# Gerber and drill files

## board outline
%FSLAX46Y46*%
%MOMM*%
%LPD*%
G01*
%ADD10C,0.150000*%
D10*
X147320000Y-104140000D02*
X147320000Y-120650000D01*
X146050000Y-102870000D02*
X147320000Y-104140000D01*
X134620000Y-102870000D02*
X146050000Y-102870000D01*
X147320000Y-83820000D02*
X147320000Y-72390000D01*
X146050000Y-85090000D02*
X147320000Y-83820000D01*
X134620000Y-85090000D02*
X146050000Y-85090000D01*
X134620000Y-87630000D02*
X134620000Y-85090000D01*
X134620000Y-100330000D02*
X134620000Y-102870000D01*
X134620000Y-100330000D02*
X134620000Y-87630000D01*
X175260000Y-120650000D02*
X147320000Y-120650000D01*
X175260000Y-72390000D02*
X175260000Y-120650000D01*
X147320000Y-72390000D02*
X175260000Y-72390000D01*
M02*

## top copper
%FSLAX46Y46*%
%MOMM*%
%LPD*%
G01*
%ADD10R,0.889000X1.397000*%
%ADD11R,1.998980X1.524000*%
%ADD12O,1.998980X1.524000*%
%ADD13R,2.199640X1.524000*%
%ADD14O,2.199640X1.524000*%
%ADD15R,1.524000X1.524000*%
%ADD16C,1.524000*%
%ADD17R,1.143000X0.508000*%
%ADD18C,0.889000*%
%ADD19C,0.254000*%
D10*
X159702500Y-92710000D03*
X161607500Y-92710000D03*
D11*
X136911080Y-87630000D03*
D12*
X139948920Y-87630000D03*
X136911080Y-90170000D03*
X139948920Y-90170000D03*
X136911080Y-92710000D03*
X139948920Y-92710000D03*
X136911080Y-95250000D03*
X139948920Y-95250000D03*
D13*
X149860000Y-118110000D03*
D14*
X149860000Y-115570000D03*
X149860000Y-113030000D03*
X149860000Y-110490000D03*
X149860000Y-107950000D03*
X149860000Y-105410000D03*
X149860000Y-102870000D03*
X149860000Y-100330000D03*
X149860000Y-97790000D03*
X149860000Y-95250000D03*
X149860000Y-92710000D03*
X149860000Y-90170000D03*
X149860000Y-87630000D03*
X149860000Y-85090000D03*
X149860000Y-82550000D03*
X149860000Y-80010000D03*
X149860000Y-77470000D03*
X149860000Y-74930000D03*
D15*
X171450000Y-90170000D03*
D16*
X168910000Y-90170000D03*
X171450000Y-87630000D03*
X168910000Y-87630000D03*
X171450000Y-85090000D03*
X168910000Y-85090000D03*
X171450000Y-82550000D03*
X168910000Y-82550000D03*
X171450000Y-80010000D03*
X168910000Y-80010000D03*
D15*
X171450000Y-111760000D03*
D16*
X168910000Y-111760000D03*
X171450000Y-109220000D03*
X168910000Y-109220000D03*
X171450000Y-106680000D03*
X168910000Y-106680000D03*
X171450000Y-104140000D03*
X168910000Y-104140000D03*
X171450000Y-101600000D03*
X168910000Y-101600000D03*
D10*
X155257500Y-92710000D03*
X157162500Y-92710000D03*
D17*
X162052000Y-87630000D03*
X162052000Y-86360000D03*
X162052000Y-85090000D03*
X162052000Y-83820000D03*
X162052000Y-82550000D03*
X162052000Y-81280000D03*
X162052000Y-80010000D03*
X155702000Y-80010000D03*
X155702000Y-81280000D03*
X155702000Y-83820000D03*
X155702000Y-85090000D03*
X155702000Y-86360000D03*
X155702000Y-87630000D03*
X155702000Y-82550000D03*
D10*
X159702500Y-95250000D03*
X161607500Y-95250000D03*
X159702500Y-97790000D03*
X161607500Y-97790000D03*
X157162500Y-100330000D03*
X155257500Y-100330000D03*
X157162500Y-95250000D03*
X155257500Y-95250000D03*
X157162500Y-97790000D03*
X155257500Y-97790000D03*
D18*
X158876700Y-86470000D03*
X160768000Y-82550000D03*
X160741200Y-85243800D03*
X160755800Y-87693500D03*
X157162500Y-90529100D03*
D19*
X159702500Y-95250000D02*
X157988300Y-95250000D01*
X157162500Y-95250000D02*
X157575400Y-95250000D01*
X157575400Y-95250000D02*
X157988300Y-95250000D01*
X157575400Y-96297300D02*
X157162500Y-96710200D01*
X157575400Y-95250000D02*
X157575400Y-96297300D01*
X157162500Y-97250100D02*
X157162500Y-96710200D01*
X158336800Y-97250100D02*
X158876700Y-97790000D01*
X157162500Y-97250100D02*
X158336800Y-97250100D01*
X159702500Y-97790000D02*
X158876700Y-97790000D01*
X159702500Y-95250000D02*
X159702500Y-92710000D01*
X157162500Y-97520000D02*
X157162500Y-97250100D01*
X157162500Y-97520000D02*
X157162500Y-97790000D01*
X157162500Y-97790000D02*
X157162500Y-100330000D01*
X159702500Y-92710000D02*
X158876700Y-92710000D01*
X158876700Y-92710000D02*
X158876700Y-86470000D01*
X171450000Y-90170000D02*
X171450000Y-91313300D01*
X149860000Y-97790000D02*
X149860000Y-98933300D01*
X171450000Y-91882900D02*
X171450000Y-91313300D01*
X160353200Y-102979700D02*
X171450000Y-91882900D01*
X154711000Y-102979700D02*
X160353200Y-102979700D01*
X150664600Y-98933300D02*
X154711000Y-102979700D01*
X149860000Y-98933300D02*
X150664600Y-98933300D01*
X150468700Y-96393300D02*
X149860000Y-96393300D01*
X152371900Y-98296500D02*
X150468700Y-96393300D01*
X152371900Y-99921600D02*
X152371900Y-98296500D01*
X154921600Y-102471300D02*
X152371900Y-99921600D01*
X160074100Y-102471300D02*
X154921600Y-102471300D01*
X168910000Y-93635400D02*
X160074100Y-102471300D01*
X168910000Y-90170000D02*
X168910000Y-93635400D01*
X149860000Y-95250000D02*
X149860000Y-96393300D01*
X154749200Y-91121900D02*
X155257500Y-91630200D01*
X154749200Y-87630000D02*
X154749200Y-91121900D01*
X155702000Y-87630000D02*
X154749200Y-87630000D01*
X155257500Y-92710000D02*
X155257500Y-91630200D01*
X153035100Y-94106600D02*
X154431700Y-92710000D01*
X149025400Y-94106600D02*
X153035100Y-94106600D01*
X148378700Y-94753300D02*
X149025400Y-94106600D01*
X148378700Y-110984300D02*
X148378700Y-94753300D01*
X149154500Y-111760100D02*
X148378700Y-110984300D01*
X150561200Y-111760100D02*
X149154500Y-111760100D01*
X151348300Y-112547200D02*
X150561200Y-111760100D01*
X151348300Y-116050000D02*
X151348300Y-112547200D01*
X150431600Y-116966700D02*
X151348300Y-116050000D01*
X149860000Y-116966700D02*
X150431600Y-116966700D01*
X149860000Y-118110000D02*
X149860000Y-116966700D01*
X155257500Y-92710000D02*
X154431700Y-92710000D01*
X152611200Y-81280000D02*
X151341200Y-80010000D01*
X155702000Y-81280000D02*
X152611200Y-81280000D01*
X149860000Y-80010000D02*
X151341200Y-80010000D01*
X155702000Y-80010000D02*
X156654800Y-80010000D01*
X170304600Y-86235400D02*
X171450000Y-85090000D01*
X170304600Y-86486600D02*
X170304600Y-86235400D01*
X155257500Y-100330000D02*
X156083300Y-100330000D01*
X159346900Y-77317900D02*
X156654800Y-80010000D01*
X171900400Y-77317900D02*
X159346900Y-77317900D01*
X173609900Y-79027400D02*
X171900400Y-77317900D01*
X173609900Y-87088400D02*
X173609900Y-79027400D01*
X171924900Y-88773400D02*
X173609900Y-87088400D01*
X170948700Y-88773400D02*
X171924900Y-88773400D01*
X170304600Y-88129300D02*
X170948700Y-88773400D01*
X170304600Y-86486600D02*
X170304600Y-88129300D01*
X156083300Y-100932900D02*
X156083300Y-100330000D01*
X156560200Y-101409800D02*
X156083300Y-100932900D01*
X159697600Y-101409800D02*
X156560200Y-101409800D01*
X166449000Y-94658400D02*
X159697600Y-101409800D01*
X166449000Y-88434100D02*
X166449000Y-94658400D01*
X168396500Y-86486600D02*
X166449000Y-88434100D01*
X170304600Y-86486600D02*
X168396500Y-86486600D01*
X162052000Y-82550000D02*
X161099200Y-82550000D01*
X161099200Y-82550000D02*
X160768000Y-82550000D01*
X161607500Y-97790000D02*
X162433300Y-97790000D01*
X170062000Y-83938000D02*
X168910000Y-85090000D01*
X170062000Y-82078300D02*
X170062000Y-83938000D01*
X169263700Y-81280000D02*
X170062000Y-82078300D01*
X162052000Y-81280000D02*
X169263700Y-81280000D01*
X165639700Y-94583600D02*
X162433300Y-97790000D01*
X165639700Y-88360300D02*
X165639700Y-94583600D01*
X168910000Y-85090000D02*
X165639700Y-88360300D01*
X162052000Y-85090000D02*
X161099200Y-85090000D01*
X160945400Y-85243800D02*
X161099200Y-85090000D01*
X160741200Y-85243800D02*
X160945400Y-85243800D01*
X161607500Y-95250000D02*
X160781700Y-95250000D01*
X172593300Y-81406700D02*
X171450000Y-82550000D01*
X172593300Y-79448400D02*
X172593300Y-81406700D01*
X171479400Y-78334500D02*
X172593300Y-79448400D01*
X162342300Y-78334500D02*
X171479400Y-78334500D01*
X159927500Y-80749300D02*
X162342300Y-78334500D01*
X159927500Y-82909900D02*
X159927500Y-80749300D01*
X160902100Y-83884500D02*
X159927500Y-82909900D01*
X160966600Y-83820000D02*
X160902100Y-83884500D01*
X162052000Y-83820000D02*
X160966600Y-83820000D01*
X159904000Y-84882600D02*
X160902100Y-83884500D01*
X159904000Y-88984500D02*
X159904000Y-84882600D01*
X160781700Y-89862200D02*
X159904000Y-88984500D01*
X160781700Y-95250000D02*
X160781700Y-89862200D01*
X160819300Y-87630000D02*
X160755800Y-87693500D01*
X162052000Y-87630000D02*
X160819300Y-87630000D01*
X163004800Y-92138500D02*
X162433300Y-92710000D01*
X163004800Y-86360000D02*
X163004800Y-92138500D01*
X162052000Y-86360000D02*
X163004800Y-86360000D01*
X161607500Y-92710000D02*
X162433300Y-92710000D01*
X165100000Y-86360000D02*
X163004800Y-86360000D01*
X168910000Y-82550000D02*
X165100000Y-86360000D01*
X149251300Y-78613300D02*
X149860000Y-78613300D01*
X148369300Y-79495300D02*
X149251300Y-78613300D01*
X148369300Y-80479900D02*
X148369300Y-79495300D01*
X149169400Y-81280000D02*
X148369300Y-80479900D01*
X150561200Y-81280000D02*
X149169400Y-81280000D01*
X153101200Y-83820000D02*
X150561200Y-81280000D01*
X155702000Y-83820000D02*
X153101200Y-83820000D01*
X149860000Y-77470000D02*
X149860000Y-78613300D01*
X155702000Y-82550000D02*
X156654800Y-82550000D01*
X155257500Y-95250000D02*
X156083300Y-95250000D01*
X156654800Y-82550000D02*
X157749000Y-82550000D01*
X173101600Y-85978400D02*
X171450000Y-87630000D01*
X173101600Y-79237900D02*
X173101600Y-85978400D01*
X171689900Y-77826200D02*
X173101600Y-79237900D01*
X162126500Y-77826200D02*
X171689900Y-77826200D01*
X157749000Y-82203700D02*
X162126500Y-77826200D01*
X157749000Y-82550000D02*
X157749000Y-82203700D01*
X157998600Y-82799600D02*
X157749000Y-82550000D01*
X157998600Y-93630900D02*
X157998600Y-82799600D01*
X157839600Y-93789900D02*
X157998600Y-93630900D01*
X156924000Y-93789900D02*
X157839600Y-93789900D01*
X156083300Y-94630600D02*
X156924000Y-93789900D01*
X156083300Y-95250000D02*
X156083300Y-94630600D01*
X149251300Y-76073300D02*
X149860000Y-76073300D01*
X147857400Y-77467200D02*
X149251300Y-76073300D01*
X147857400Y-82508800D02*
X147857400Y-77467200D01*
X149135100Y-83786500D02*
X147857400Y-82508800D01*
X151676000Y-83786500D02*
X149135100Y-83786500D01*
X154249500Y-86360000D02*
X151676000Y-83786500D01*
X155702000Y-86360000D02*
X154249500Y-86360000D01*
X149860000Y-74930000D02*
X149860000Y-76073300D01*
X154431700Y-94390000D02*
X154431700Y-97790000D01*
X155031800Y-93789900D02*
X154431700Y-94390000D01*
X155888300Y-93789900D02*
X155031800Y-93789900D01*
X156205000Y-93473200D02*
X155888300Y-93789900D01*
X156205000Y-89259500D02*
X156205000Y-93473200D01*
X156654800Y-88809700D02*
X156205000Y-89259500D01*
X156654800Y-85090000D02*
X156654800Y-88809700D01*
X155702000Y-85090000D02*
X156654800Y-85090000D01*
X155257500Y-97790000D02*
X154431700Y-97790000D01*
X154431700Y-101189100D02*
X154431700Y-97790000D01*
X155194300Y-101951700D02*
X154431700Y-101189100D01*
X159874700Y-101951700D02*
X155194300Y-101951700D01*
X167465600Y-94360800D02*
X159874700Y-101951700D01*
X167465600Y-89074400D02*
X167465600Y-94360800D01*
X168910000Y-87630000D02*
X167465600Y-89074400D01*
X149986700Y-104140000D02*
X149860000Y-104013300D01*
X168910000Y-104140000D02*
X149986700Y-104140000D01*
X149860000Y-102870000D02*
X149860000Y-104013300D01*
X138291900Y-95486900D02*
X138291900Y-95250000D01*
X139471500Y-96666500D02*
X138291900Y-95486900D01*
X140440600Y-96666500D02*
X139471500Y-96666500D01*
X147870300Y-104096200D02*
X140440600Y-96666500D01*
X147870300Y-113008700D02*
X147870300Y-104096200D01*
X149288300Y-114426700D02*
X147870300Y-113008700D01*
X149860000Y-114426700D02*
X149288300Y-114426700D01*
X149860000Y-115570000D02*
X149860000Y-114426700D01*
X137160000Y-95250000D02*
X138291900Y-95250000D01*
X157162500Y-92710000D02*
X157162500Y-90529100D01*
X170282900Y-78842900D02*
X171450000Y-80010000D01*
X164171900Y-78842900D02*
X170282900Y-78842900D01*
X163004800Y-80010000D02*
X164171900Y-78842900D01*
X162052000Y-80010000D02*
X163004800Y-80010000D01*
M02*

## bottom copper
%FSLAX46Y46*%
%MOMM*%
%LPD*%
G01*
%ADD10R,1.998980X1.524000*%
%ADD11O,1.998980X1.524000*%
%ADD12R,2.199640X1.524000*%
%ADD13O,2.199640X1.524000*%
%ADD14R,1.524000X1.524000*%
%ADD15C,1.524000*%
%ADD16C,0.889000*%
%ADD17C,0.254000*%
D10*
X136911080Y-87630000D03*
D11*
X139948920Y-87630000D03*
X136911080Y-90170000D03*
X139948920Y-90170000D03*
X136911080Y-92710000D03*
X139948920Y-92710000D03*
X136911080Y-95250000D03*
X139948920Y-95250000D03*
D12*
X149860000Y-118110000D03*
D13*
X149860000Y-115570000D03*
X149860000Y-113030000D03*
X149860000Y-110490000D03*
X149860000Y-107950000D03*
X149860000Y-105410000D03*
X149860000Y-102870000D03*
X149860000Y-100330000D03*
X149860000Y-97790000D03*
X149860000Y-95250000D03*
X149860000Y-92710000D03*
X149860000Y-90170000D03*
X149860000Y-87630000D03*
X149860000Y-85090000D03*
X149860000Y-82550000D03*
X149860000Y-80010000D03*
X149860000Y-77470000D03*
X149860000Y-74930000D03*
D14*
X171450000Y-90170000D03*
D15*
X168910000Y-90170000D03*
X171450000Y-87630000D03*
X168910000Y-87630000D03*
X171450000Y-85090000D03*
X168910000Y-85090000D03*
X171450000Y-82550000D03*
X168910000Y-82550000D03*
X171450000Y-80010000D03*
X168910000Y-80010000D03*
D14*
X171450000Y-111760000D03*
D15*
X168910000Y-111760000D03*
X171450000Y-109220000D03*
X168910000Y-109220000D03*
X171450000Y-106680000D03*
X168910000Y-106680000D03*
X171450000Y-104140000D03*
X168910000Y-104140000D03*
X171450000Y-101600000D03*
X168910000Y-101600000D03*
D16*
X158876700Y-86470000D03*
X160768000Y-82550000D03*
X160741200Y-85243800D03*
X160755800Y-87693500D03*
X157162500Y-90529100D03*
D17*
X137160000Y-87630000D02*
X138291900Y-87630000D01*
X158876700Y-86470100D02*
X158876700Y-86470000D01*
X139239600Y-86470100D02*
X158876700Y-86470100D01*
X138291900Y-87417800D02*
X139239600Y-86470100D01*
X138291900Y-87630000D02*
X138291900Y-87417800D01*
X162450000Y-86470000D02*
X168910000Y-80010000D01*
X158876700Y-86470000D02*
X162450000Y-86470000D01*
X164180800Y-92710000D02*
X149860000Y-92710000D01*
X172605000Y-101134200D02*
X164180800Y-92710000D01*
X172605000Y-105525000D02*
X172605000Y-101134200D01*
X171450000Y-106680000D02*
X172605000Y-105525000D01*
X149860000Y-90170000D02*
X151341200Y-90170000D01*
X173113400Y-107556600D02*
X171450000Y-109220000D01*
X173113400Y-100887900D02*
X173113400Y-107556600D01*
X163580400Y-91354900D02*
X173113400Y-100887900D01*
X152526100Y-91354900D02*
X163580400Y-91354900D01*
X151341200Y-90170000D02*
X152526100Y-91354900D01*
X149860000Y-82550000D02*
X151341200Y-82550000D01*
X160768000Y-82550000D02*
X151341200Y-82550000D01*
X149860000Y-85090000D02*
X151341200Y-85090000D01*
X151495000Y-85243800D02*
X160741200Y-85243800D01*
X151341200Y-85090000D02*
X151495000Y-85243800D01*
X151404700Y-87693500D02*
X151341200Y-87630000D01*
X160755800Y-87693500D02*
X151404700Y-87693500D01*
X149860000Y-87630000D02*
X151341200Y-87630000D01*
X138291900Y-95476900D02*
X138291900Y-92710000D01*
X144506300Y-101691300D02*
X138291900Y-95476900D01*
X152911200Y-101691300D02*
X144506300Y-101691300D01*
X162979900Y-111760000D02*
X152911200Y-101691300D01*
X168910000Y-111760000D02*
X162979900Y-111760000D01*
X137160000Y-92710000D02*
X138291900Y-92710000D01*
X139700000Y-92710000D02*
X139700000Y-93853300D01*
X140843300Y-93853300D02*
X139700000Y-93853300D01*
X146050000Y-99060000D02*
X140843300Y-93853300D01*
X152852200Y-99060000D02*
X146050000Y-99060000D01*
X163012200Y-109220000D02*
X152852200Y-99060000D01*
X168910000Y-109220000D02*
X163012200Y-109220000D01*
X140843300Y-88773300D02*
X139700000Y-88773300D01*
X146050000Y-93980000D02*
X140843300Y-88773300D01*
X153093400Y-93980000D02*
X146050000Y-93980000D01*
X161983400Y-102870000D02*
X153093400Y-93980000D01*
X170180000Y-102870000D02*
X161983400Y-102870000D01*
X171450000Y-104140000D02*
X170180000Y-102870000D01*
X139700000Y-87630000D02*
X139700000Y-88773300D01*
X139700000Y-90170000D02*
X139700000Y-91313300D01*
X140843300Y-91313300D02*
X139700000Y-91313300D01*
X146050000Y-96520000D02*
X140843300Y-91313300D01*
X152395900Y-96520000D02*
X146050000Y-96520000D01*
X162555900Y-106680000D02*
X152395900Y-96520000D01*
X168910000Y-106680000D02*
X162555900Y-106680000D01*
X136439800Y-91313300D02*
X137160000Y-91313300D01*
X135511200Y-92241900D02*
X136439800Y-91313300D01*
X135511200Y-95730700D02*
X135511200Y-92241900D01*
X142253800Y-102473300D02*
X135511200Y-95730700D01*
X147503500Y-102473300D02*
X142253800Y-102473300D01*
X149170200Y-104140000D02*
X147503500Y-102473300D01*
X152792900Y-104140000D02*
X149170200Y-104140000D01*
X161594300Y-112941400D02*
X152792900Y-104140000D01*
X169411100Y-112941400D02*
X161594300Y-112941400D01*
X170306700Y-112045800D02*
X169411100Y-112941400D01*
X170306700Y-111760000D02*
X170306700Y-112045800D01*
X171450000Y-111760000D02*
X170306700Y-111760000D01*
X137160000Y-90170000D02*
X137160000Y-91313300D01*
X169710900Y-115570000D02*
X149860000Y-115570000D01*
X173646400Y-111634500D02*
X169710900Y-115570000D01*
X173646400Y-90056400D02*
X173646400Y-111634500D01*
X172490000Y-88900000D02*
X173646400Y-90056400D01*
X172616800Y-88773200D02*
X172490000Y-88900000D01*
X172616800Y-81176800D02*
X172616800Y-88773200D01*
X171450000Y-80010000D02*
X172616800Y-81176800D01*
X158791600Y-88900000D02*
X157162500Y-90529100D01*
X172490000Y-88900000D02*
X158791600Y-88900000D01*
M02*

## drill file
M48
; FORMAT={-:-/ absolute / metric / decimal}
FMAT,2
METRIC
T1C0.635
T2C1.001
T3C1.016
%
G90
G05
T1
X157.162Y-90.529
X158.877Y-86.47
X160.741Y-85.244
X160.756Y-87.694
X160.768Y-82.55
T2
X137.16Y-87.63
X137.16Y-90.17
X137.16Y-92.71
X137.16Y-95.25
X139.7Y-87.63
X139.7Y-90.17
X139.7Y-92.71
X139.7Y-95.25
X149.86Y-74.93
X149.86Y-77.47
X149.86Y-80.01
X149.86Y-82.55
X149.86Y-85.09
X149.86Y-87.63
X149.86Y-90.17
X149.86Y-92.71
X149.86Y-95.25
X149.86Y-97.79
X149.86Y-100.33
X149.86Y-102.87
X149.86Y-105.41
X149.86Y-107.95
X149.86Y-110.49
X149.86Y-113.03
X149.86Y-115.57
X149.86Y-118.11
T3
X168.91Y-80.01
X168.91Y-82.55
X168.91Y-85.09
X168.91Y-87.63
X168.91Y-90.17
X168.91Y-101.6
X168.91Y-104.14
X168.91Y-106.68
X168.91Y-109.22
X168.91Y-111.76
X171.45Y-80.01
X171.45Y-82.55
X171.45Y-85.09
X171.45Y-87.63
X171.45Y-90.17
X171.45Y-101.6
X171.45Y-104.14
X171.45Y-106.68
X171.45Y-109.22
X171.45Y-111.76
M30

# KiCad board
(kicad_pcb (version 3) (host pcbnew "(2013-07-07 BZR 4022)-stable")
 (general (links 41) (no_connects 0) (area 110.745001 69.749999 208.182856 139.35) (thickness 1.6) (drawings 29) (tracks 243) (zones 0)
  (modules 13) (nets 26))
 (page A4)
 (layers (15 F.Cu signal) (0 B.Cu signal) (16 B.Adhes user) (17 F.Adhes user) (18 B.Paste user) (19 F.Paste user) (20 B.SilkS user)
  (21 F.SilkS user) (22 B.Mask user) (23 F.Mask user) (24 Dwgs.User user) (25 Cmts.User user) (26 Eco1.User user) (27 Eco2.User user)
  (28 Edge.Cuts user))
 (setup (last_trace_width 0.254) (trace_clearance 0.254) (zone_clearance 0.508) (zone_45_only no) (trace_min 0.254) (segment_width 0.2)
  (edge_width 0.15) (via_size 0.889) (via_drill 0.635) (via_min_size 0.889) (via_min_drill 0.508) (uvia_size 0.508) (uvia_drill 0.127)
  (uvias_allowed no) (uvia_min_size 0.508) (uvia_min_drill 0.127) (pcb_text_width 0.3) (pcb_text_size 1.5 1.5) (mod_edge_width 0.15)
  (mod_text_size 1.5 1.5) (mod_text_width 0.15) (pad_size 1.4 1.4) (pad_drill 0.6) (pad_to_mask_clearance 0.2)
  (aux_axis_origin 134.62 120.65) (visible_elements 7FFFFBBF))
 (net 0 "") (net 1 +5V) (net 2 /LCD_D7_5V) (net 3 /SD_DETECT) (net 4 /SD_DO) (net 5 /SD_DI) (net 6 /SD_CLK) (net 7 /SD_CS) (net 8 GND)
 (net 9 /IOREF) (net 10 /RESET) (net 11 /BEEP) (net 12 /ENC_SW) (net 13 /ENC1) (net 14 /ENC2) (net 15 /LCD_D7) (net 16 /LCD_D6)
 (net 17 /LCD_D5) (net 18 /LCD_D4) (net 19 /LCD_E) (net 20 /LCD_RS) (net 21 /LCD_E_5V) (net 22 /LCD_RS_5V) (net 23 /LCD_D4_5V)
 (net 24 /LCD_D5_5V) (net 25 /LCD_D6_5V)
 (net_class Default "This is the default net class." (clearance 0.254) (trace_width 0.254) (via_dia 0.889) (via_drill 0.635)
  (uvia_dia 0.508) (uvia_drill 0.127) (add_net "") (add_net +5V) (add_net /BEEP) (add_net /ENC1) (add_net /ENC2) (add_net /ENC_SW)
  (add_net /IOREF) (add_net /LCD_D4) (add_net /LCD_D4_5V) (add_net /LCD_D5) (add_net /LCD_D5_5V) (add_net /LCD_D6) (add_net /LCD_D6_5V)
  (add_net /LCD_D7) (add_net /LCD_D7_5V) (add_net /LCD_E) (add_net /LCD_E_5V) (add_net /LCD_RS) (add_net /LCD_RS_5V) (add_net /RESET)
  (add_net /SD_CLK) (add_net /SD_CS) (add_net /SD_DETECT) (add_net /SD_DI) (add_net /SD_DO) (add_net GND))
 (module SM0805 (layer F.Cu) (at 160.655 92.71)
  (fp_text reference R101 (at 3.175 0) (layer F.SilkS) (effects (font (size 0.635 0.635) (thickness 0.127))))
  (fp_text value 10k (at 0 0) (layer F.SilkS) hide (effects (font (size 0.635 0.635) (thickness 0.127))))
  (pad 1 smd rect (at -0.9525 0) (size 0.889 1.397) (layers F.Cu F.Paste F.Mask) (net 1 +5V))
  (pad 2 smd rect (at 0.9525 0) (size 0.889 1.397) (layers F.Cu F.Paste F.Mask) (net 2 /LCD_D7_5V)))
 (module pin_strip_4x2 (layer F.Cu) (at 138.43 91.44 270)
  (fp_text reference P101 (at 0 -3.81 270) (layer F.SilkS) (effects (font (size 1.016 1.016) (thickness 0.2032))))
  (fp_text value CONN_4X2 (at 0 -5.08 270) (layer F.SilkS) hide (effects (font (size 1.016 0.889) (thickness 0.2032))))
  (pad 1 thru_hole rect (at -3.81 1.27 270) (size 1.524 1.99898) (drill 1.00076 (offset 0 0.24892)) (layers *.Cu *.Mask F.SilkS) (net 1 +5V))
  (pad 2 thru_hole oval (at -3.81 -1.27 270) (size 1.524 1.99898) (drill 1.00076 (offset 0 -0.24892)) (layers *.Cu *.Mask F.SilkS)
   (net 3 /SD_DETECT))
  (pad 3 thru_hole oval (at -1.27 1.27 270) (size 1.524 1.99898) (drill 1.00076 (offset 0 0.24892)) (layers *.Cu *.Mask F.SilkS)
   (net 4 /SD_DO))
  (pad 4 thru_hole oval (at -1.27 -1.27 270) (size 1.524 1.99898) (drill 1.00076 (offset 0 -0.24892)) (layers *.Cu *.Mask F.SilkS)
   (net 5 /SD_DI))
  (pad 5 thru_hole oval (at 1.27 1.27 270) (size 1.524 1.99898) (drill 1.00076 (offset 0 0.24892)) (layers *.Cu *.Mask F.SilkS)
   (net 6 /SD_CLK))
  (pad 6 thru_hole oval (at 1.27 -1.27 270) (size 1.524 1.99898) (drill 1.00076 (offset 0 -0.24892)) (layers *.Cu *.Mask F.SilkS)
   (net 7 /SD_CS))
  (pad 7 thru_hole oval (at 3.81 1.27 270) (size 1.524 1.99898) (drill 1.00076 (offset 0 0.24892)) (layers *.Cu *.Mask F.SilkS) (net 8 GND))
  (pad 8 thru_hole oval (at 3.81 -1.27 270) (size 1.524 1.99898) (drill 1.00076 (offset 0 -0.24892)) (layers *.Cu *.Mask F.SilkS)))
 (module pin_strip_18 (layer B.Cu) (at 149.86 96.52 90)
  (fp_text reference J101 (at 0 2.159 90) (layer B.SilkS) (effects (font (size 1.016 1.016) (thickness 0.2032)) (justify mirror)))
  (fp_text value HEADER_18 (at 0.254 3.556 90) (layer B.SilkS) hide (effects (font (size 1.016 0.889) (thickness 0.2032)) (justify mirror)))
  (pad 1 thru_hole rect (at -21.59 0 90) (size 1.524 2.19964) (drill 1.00076) (layers *.Cu *.Mask B.SilkS) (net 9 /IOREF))
  (pad 2 thru_hole oval (at -19.05 0 90) (size 1.524 2.19964) (drill 1.00076) (layers *.Cu *.Mask B.SilkS) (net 8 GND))
  (pad 3 thru_hole oval (at -16.51 0 90) (size 1.524 2.19964) (drill 1.00076) (layers *.Cu *.Mask B.SilkS))
  (pad 4 thru_hole oval (at -13.97 0 90) (size 1.524 2.19964) (drill 1.00076) (layers *.Cu *.Mask B.SilkS))
  (pad 5 thru_hole oval (at -11.43 0 90) (size 1.524 2.19964) (drill 1.00076) (layers *.Cu *.Mask B.SilkS))
  (pad 6 thru_hole oval (at -8.89 0 90) (size 1.524 2.19964) (drill 1.00076) (layers *.Cu *.Mask B.SilkS))
  (pad 7 thru_hole oval (at -6.35 0 90) (size 1.524 2.19964) (drill 1.00076) (layers *.Cu *.Mask B.SilkS) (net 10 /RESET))
  (pad 8 thru_hole oval (at -3.81 0 90) (size 1.524 2.19964) (drill 1.00076) (layers *.Cu *.Mask B.SilkS))
  (pad 9 thru_hole oval (at -1.27 0 90) (size 1.524 2.19964) (drill 1.00076) (layers *.Cu *.Mask B.SilkS) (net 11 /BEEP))
  (pad 10 thru_hole oval (at 1.27 0 90) (size 1.524 2.19964) (drill 1.00076) (layers *.Cu *.Mask B.SilkS) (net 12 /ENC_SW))
  (pad 11 thru_hole oval (at 3.81 0 90) (size 1.524 2.19964) (drill 1.00076) (layers *.Cu *.Mask B.SilkS) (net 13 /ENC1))
  (pad 12 thru_hole oval (at 6.35 0 90) (size 1.524 2.19964) (drill 1.00076) (layers *.Cu *.Mask B.SilkS) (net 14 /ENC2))
  (pad 13 thru_hole oval (at 8.89 0 90) (size 1.524 2.19964) (drill 1.00076) (layers *.Cu *.Mask B.SilkS) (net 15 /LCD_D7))
  (pad 14 thru_hole oval (at 11.43 0 90) (size 1.524 2.19964) (drill 1.00076) (layers *.Cu *.Mask B.SilkS) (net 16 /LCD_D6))
  (pad 15 thru_hole oval (at 13.97 0 90) (size 1.524 2.19964) (drill 1.00076) (layers *.Cu *.Mask B.SilkS) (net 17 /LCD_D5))
  (pad 16 thru_hole oval (at 16.51 0 90) (size 1.524 2.19964) (drill 1.00076) (layers *.Cu *.Mask B.SilkS) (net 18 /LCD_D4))
  (pad 17 thru_hole oval (at 19.05 0 90) (size 1.524 2.19964) (drill 1.00076) (layers *.Cu *.Mask B.SilkS) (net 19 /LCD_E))
  (pad 18 thru_hole oval (at 21.59 0 90) (size 1.524 2.19964) (drill 1.00076) (layers *.Cu *.Mask B.SilkS) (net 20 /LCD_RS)))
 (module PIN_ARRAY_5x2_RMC (layer F.Cu) (at 170.18 85.09 90)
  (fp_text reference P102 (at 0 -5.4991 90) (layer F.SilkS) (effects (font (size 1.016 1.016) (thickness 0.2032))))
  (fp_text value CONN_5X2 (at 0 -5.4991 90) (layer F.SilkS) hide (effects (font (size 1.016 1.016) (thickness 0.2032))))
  (pad 1 thru_hole rect (at -5.08 1.27 90) (size 1.524 1.524) (drill 1.016) (layers *.Cu *.Mask F.SilkS) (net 11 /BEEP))
  (pad 2 thru_hole circle (at -5.08 -1.27 90) (size 1.524 1.524) (drill 1.016) (layers *.Cu *.Mask F.SilkS) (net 12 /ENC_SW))
  (pad 3 thru_hole circle (at -2.54 1.27 90) (size 1.524 1.524) (drill 1.016) (layers *.Cu *.Mask F.SilkS) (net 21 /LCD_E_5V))
  (pad 4 thru_hole circle (at -2.54 -1.27 90) (size 1.524 1.524) (drill 1.016) (layers *.Cu *.Mask F.SilkS) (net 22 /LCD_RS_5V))
  (pad 5 thru_hole circle (at 0 1.27 90) (size 1.524 1.524) (drill 1.016) (layers *.Cu *.Mask F.SilkS) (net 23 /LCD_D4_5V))
  (pad 6 thru_hole circle (at 0 -1.27 90) (size 1.524 1.524) (drill 1.016) (layers *.Cu *.Mask F.SilkS) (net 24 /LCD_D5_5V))
  (pad 7 thru_hole circle (at 2.54 1.27 90) (size 1.524 1.524) (drill 1.016) (layers *.Cu *.Mask F.SilkS) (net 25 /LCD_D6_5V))
  (pad 8 thru_hole circle (at 2.54 -1.27 90) (size 1.524 1.524) (drill 1.016) (layers *.Cu *.Mask F.SilkS) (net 2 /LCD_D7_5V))
  (pad 9 thru_hole circle (at 5.08 1.27 90) (size 1.524 1.524) (drill 1.016) (layers *.Cu *.Mask F.SilkS) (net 8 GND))
  (pad 10 thru_hole circle (at 5.08 -1.27 90) (size 1.524 1.524) (drill 1.016) (layers *.Cu *.Mask F.SilkS) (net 1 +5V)))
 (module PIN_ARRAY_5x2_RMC (layer F.Cu) (at 170.18 106.68 90)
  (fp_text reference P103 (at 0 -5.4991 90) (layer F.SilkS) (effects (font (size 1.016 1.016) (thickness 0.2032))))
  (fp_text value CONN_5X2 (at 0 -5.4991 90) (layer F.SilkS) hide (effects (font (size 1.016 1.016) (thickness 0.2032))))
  (pad 1 thru_hole rect (at -5.08 1.27 90) (size 1.524 1.524) (drill 1.016) (layers *.Cu *.Mask F.SilkS) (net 4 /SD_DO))
  (pad 2 thru_hole circle (at -5.08 -1.27 90) (size 1.524 1.524) (drill 1.016) (layers *.Cu *.Mask F.SilkS) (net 6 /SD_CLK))
  (pad 3 thru_hole circle (at -2.54 1.27 90) (size 1.524 1.524) (drill 1.016) (layers *.Cu *.Mask F.SilkS) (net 14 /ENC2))
  (pad 4 thru_hole circle (at -2.54 -1.27 90) (size 1.524 1.524) (drill 1.016) (layers *.Cu *.Mask F.SilkS) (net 7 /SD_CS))
  (pad 5 thru_hole circle (at 0 1.27 90) (size 1.524 1.524) (drill 1.016) (layers *.Cu *.Mask F.SilkS) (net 13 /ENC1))
  (pad 6 thru_hole circle (at 0 -1.27 90) (size 1.524 1.524) (drill 1.016) (layers *.Cu *.Mask F.SilkS) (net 5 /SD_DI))
  (pad 7 thru_hole circle (at 2.54 1.27 90) (size 1.524 1.524) (drill 1.016) (layers *.Cu *.Mask F.SilkS) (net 3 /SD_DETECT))
  (pad 8 thru_hole circle (at 2.54 -1.27 90) (size 1.524 1.524) (drill 1.016) (layers *.Cu *.Mask F.SilkS) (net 10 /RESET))
  (pad 9 thru_hole circle (at 5.08 1.27 90) (size 1.524 1.524) (drill 1.016) (layers *.Cu *.Mask F.SilkS))
  (pad 10 thru_hole circle (at 5.08 -1.27 90) (size 1.524 1.524) (drill 1.016) (layers *.Cu *.Mask F.SilkS)))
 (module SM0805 (layer F.Cu) (at 156.21 92.71)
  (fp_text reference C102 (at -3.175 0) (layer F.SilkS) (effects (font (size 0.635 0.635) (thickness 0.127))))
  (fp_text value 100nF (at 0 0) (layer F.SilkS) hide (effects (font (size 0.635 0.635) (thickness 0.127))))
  (pad 1 smd rect (at -0.9525 0) (size 0.889 1.397) (layers F.Cu F.Paste F.Mask) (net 9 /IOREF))
  (pad 2 smd rect (at 0.9525 0) (size 0.889 1.397) (layers F.Cu F.Paste F.Mask) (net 8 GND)))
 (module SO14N (layer F.Cu) (at 158.75 83.82 90)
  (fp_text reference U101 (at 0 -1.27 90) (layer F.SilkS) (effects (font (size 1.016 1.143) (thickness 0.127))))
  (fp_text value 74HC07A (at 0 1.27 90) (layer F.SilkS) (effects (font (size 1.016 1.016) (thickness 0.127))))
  (pad 1 smd rect (at -3.81 3.302 90) (size 0.508 1.143) (layers F.Cu F.Paste F.Mask) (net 15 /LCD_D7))
  (pad 2 smd rect (at -2.54 3.302 90) (size 0.508 1.143) (layers F.Cu F.Paste F.Mask) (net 2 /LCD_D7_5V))
  (pad 3 smd rect (at -1.27 3.302 90) (size 0.508 1.143) (layers F.Cu F.Paste F.Mask) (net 16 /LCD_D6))
  (pad 4 smd rect (at 0 3.302 90) (size 0.508 1.143) (layers F.Cu F.Paste F.Mask) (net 25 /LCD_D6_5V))
  (pad 5 smd rect (at 1.27 3.302 90) (size 0.508 1.143) (layers F.Cu F.Paste F.Mask) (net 17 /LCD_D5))
  (pad 6 smd rect (at 2.54 3.302 90) (size 0.508 1.143) (layers F.Cu F.Paste F.Mask) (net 24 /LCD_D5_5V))
  (pad 7 smd rect (at 3.81 3.302 90) (size 0.508 1.143) (layers F.Cu F.Paste F.Mask) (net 8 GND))
  (pad 8 smd rect (at 3.81 -3.048 90) (size 0.508 1.143) (layers F.Cu F.Paste F.Mask) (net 23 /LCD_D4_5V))
  (pad 9 smd rect (at 2.54 -3.048 90) (size 0.508 1.143) (layers F.Cu F.Paste F.Mask) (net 18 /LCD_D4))
  (pad 11 smd rect (at 0 -3.048 90) (size 0.508 1.143) (layers F.Cu F.Paste F.Mask) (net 19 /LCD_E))
  (pad 12 smd rect (at -1.27 -3.048 90) (size 0.508 1.143) (layers F.Cu F.Paste F.Mask) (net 22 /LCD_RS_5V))
  (pad 13 smd rect (at -2.54 -3.048 90) (size 0.508 1.143) (layers F.Cu F.Paste F.Mask) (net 20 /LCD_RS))
  (pad 14 smd rect (at -3.81 -3.048 90) (size 0.508 1.143) (layers F.Cu F.Paste F.Mask) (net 9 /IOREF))
  (pad 10 smd rect (at 1.27 -3.048 90) (size 0.508 1.143) (layers F.Cu F.Paste F.Mask) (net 21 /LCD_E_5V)))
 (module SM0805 (layer F.Cu) (at 160.655 95.25)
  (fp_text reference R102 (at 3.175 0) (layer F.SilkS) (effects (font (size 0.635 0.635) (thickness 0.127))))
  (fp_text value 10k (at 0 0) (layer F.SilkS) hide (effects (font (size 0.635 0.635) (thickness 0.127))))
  (pad 1 smd rect (at -0.9525 0) (size 0.889 1.397) (layers F.Cu F.Paste F.Mask) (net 1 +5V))
  (pad 2 smd rect (at 0.9525 0) (size 0.889 1.397) (layers F.Cu F.Paste F.Mask) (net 25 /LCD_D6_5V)))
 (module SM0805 (layer F.Cu) (at 160.655 97.79)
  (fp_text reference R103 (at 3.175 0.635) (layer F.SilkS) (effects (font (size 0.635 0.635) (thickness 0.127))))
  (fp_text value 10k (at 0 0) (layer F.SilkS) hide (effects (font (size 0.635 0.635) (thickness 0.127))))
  (pad 1 smd rect (at -0.9525 0) (size 0.889 1.397) (layers F.Cu F.Paste F.Mask) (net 1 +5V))
  (pad 2 smd rect (at 0.9525 0) (size 0.889 1.397) (layers F.Cu F.Paste F.Mask) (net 24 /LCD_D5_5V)))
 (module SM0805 (layer F.Cu) (at 156.21 100.33 180)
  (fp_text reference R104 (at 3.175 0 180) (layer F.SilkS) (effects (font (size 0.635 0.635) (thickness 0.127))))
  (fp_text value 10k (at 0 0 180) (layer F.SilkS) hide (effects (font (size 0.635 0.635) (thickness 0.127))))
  (pad 1 smd rect (at -0.9525 0 180) (size 0.889 1.397) (layers F.Cu F.Paste F.Mask) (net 1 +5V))
  (pad 2 smd rect (at 0.9525 0 180) (size 0.889 1.397) (layers F.Cu F.Paste F.Mask) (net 23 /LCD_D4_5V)))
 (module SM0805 (layer F.Cu) (at 156.21 95.25 180)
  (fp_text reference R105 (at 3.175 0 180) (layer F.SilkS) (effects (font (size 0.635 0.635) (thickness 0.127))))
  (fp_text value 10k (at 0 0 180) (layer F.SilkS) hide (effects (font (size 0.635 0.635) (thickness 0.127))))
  (pad 1 smd rect (at -0.9525 0 180) (size 0.889 1.397) (layers F.Cu F.Paste F.Mask) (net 1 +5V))
  (pad 2 smd rect (at 0.9525 0 180) (size 0.889 1.397) (layers F.Cu F.Paste F.Mask) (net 21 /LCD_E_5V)))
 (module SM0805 (layer F.Cu) (at 156.21 97.79 180)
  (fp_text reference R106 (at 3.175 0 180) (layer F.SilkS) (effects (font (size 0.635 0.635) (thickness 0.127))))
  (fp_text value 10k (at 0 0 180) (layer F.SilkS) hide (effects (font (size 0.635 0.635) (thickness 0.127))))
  (pad 1 smd rect (at -0.9525 0 180) (size 0.889 1.397) (layers F.Cu F.Paste F.Mask) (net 1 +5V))
  (pad 2 smd rect (at 0.9525 0 180) (size 0.889 1.397) (layers F.Cu F.Paste F.Mask) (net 22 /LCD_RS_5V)))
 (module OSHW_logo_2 (layer F.Cu) (at 158.75 110.49)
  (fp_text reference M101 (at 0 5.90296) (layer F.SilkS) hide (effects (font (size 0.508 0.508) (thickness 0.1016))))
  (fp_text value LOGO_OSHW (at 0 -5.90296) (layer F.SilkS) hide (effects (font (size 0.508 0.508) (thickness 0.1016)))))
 (gr_line (start 147.32 104.14) (end 147.32 120.65) (angle 90) (layer Edge.Cuts) (width 0.15))
 (gr_line (start 146.05 102.87) (end 147.32 104.14) (angle 90) (layer Edge.Cuts) (width 0.15))
 (gr_line (start 134.62 102.87) (end 146.05 102.87) (angle 90) (layer Edge.Cuts) (width 0.15))
 (gr_line (start 147.32 83.82) (end 147.32 72.39) (angle 90) (layer Edge.Cuts) (width 0.15))
 (gr_line (start 146.05 85.09) (end 147.32 83.82) (angle 90) (layer Edge.Cuts) (width 0.15))
 (gr_line (start 134.62 85.09) (end 146.05 85.09) (angle 90) (layer Edge.Cuts) (width 0.15))
 (gr_line (start 134.62 87.63) (end 134.62 85.09) (angle 90) (layer Edge.Cuts) (width 0.15))
 (gr_line (start 134.62 100.33) (end 134.62 102.87) (angle 90) (layer Edge.Cuts) (width 0.15))
 (gr_line (start 134.62 100.33) (end 134.62 87.63) (angle 90) (layer Edge.Cuts) (width 0.15))
 (gr_line (start 175.26 120.65) (end 147.32 120.65) (angle 90) (layer Edge.Cuts) (width 0.15))
 (gr_line (start 175.26 72.39) (end 175.26 120.65) (angle 90) (layer Edge.Cuts) (width 0.15))
 (gr_line (start 147.32 72.39) (end 175.26 72.39) (angle 90) (layer Edge.Cuts) (width 0.15))
 (via (at 158.8767 86.47) (size 0.889) (layers F.Cu B.Cu) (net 1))
 (segment (start 159.7025 95.25) (end 157.9883 95.25) (width 0.254) (layer F.Cu) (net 1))
 (segment (start 157.1625 95.25) (end 157.5754 95.25) (width 0.254) (layer F.Cu) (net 1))
 (segment (start 157.5754 95.25) (end 157.9883 95.25) (width 0.254) (layer F.Cu) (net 1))
 (segment (start 157.5754 96.2973) (end 157.1625 96.7102) (width 0.254) (layer F.Cu) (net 1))
 (segment (start 157.5754 95.25) (end 157.5754 96.2973) (width 0.254) (layer F.Cu) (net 1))
 (segment (start 157.1625 97.2501) (end 157.1625 96.7102) (width 0.254) (layer F.Cu) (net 1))
 (segment (start 158.3368 97.2501) (end 158.8767 97.79) (width 0.254) (layer F.Cu) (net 1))
 (segment (start 157.1625 97.2501) (end 158.3368 97.2501) (width 0.254) (layer F.Cu) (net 1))
 (segment (start 159.7025 97.79) (end 158.8767 97.79) (width 0.254) (layer F.Cu) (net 1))
 (segment (start 159.7025 95.25) (end 159.7025 92.71) (width 0.254) (layer F.Cu) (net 1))
 (segment (start 157.1625 97.52) (end 157.1625 97.2501) (width 0.254) (layer F.Cu) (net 1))
 (segment (start 157.1625 97.52) (end 157.1625 97.79) (width 0.254) (layer F.Cu) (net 1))
 (segment (start 157.1625 97.79) (end 157.1625 100.33) (width 0.254) (layer F.Cu) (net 1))
 (segment (start 137.16 87.63) (end 138.2919 87.63) (width 0.254) (layer B.Cu) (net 1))
 (segment (start 159.7025 92.71) (end 158.8767 92.71) (width 0.254) (layer F.Cu) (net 1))
 (segment (start 158.8767 86.4701) (end 158.8767 86.47) (width 0.254) (layer B.Cu) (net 1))
 (segment (start 139.2396 86.4701) (end 158.8767 86.4701) (width 0.254) (layer B.Cu) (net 1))
 (segment (start 138.2919 87.4178) (end 139.2396 86.4701) (width 0.254) (layer B.Cu) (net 1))
 (segment (start 138.2919 87.63) (end 138.2919 87.4178) (width 0.254) (layer B.Cu) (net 1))
 (segment (start 162.45 86.47) (end 168.91 80.01) (width 0.254) (layer B.Cu) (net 1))
 (segment (start 158.8767 86.47) (end 162.45 86.47) (width 0.254) (layer B.Cu) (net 1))
 (segment (start 158.8767 92.71) (end 158.8767 86.47) (width 0.254) (layer F.Cu) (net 1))
 (segment (start 171.45 90.17) (end 171.45 91.3133) (width 0.254) (layer F.Cu) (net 11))
 (segment (start 149.86 97.79) (end 149.86 98.9333) (width 0.254) (layer F.Cu) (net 11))
 (segment (start 171.45 91.8829) (end 171.45 91.3133) (width 0.254) (layer F.Cu) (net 11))
 (segment (start 160.3532 102.9797) (end 171.45 91.8829) (width 0.254) (layer F.Cu) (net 11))
 (segment (start 154.711 102.9797) (end 160.3532 102.9797) (width 0.254) (layer F.Cu) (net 11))
 (segment (start 150.6646 98.9333) (end 154.711 102.9797) (width 0.254) (layer F.Cu) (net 11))
 (segment (start 149.86 98.9333) (end 150.6646 98.9333) (width 0.254) (layer F.Cu) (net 11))
 (segment (start 164.1808 92.71) (end 149.86 92.71) (width 0.254) (layer B.Cu) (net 13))
 (segment (start 172.605 101.1342) (end 164.1808 92.71) (width 0.254) (layer B.Cu) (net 13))
 (segment (start 172.605 105.525) (end 172.605 101.1342) (width 0.254) (layer B.Cu) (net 13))
 (segment (start 171.45 106.68) (end 172.605 105.525) (width 0.254) (layer B.Cu) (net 13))
 (segment (start 149.86 90.17) (end 151.3412 90.17) (width 0.254) (layer B.Cu) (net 14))
 (segment (start 173.1134 107.5566) (end 171.45 109.22) (width 0.254) (layer B.Cu) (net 14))
 (segment (start 173.1134 100.8879) (end 173.1134 107.5566) (width 0.254) (layer B.Cu) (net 14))
 (segment (start 163.5804 91.3549) (end 173.1134 100.8879) (width 0.254) (layer B.Cu) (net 14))
 (segment (start 152.5261 91.3549) (end 163.5804 91.3549) (width 0.254) (layer B.Cu) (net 14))
 (segment (start 151.3412 90.17) (end 152.5261 91.3549) (width 0.254) (layer B.Cu) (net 14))
 (segment (start 150.4687 96.3933) (end 149.86 96.3933) (width 0.254) (layer F.Cu) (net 12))
 (segment (start 152.3719 98.2965) (end 150.4687 96.3933) (width 0.254) (layer F.Cu) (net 12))
 (segment (start 152.3719 99.9216) (end 152.3719 98.2965) (width 0.254) (layer F.Cu) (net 12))
 (segment (start 154.9216 102.4713) (end 152.3719 99.9216) (width 0.254) (layer F.Cu) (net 12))
 (segment (start 160.0741 102.4713) (end 154.9216 102.4713) (width 0.254) (layer F.Cu) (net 12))
 (segment (start 168.91 93.6354) (end 160.0741 102.4713) (width 0.254) (layer F.Cu) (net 12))
 (segment (start 168.91 90.17) (end 168.91 93.6354) (width 0.254) (layer F.Cu) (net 12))
 (segment (start 149.86 95.25) (end 149.86 96.3933) (width 0.254) (layer F.Cu) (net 12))
 (segment (start 154.7492 91.1219) (end 155.2575 91.6302) (width 0.254) (layer F.Cu) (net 9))
 (segment (start 154.7492 87.63) (end 154.7492 91.1219) (width 0.254) (layer F.Cu) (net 9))
 (segment (start 155.702 87.63) (end 154.7492 87.63) (width 0.254) (layer F.Cu) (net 9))
 (segment (start 155.2575 92.71) (end 155.2575 91.6302) (width 0.254) (layer F.Cu) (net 9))
 (segment (start 153.0351 94.1066) (end 154.4317 92.71) (width 0.254) (layer F.Cu) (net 9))
 (segment (start 149.0254 94.1066) (end 153.0351 94.1066) (width 0.254) (layer F.Cu) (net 9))
 (segment (start 148.3787 94.7533) (end 149.0254 94.1066) (width 0.254) (layer F.Cu) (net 9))
 (segment (start 148.3787 110.9843) (end 148.3787 94.7533) (width 0.254) (layer F.Cu) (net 9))
 (segment (start 149.1545 111.7601) (end 148.3787 110.9843) (width 0.254) (layer F.Cu) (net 9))
 (segment (start 150.5612 111.7601) (end 149.1545 111.7601) (width 0.254) (layer F.Cu) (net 9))
 (segment (start 151.3483 112.5472) (end 150.5612 111.7601) (width 0.254) (layer F.Cu) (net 9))
 (segment (start 151.3483 116.05) (end 151.3483 112.5472) (width 0.254) (layer F.Cu) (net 9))
 (segment (start 150.4316 116.9667) (end 151.3483 116.05) (width 0.254) (layer F.Cu) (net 9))
 (segment (start 149.86 116.9667) (end 150.4316 116.9667) (width 0.254) (layer F.Cu) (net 9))
 (segment (start 149.86 118.11) (end 149.86 116.9667) (width 0.254) (layer F.Cu) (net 9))
 (segment (start 155.2575 92.71) (end 154.4317 92.71) (width 0.254) (layer F.Cu) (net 9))
 (segment (start 152.6112 81.28) (end 151.3412 80.01) (width 0.254) (layer F.Cu) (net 18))
 (segment (start 155.702 81.28) (end 152.6112 81.28) (width 0.254) (layer F.Cu) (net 18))
 (segment (start 149.86 80.01) (end 151.3412 80.01) (width 0.254) (layer F.Cu) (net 18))
 (segment (start 155.702 80.01) (end 156.6548 80.01) (width 0.254) (layer F.Cu) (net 23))
 (segment (start 170.3046 86.2354) (end 171.45 85.09) (width 0.254) (layer F.Cu) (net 23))
 (segment (start 170.3046 86.4866) (end 170.3046 86.2354) (width 0.254) (layer F.Cu) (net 23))
 (segment (start 155.2575 100.33) (end 156.0833 100.33) (width 0.254) (layer F.Cu) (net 23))
 (segment (start 159.3469 77.3179) (end 156.6548 80.01) (width 0.254) (layer F.Cu) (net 23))
 (segment (start 171.9004 77.3179) (end 159.3469 77.3179) (width 0.254) (layer F.Cu) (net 23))
 (segment (start 173.6099 79.0274) (end 171.9004 77.3179) (width 0.254) (layer F.Cu) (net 23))
 (segment (start 173.6099 87.0884) (end 173.6099 79.0274) (width 0.254) (layer F.Cu) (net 23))
 (segment (start 171.9249 88.7734) (end 173.6099 87.0884) (width 0.254) (layer F.Cu) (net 23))
 (segment (start 170.9487 88.7734) (end 171.9249 88.7734) (width 0.254) (layer F.Cu) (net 23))
 (segment (start 170.3046 88.1293) (end 170.9487 88.7734) (width 0.254) (layer F.Cu) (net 23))
 (segment (start 170.3046 86.4866) (end 170.3046 88.1293) (width 0.254) (layer F.Cu) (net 23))
 (segment (start 156.0833 100.9329) (end 156.0833 100.33) (width 0.254) (layer F.Cu) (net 23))
 (segment (start 156.5602 101.4098) (end 156.0833 100.9329) (width 0.254) (layer F.Cu) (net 23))
 (segment (start 159.6976 101.4098) (end 156.5602 101.4098) (width 0.254) (layer F.Cu) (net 23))
 (segment (start 166.449 94.6584) (end 159.6976 101.4098) (width 0.254) (layer F.Cu) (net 23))
 (segment (start 166.449 88.4341) (end 166.449 94.6584) (width 0.254) (layer F.Cu) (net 23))
 (segment (start 168.3965 86.4866) (end 166.449 88.4341) (width 0.254) (layer F.Cu) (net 23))
 (segment (start 170.3046 86.4866) (end 168.3965 86.4866) (width 0.254) (layer F.Cu) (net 23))
 (via (at 160.768 82.55) (size 0.889) (layers F.Cu B.Cu) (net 17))
 (segment (start 149.86 82.55) (end 151.3412 82.55) (width 0.254) (layer B.Cu) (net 17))
 (segment (start 162.052 82.55) (end 161.0992 82.55) (width 0.254) (layer F.Cu) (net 17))
 (segment (start 161.0992 82.55) (end 160.768 82.55) (width 0.254) (layer F.Cu) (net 17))
 (segment (start 160.768 82.55) (end 151.3412 82.55) (width 0.254) (layer B.Cu) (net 17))
 (segment (start 161.6075 97.79) (end 162.4333 97.79) (width 0.254) (layer F.Cu) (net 24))
 (segment (start 170.062 83.938) (end 168.91 85.09) (width 0.254) (layer F.Cu) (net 24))
 (segment (start 170.062 82.0783) (end 170.062 83.938) (width 0.254) (layer F.Cu) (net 24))
 (segment (start 169.2637 81.28) (end 170.062 82.0783) (width 0.254) (layer F.Cu) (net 24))
 (segment (start 162.052 81.28) (end 169.2637 81.28) (width 0.254) (layer F.Cu) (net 24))
 (segment (start 165.6397 94.5836) (end 162.4333 97.79) (width 0.254) (layer F.Cu) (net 24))
 (segment (start 165.6397 88.3603) (end 165.6397 94.5836) (width 0.254) (layer F.Cu) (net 24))
 (segment (start 168.91 85.09) (end 165.6397 88.3603) (width 0.254) (layer F.Cu) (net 24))
 (via (at 160.7412 85.2438) (size 0.889) (layers F.Cu B.Cu) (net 16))
 (segment (start 149.86 85.09) (end 151.3412 85.09) (width 0.254) (layer B.Cu) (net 16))
 (segment (start 162.052 85.09) (end 161.0992 85.09) (width 0.254) (layer F.Cu) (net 16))
 (segment (start 160.9454 85.2438) (end 161.0992 85.09) (width 0.254) (layer F.Cu) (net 16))
 (segment (start 160.7412 85.2438) (end 160.9454 85.2438) (width 0.254) (layer F.Cu) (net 16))
 (segment (start 151.495 85.2438) (end 160.7412 85.2438) (width 0.254) (layer B.Cu) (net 16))
 (segment (start 151.3412 85.09) (end 151.495 85.2438) (width 0.254) (layer B.Cu) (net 16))
 (segment (start 161.6075 95.25) (end 160.7817 95.25) (width 0.254) (layer F.Cu) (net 25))
 (segment (start 172.5933 81.4067) (end 171.45 82.55) (width 0.254) (layer F.Cu) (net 25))
 (segment (start 172.5933 79.4484) (end 172.5933 81.4067) (width 0.254) (layer F.Cu) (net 25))
 (segment (start 171.4794 78.3345) (end 172.5933 79.4484) (width 0.254) (layer F.Cu) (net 25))
 (segment (start 162.3423 78.3345) (end 171.4794 78.3345) (width 0.254) (layer F.Cu) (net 25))
 (segment (start 159.9275 80.7493) (end 162.3423 78.3345) (width 0.254) (layer F.Cu) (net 25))
 (segment (start 159.9275 82.9099) (end 159.9275 80.7493) (width 0.254) (layer F.Cu) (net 25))
 (segment (start 160.9021 83.8845) (end 159.9275 82.9099) (width 0.254) (layer F.Cu) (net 25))
 (segment (start 160.9666 83.82) (end 160.9021 83.8845) (width 0.254) (layer F.Cu) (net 25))
 (segment (start 162.052 83.82) (end 160.9666 83.82) (width 0.254) (layer F.Cu) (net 25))
 (segment (start 159.904 84.8826) (end 160.9021 83.8845) (width 0.254) (layer F.Cu) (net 25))
 (segment (start 159.904 88.9845) (end 159.904 84.8826) (width 0.254) (layer F.Cu) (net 25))
 (segment (start 160.7817 89.8622) (end 159.904 88.9845) (width 0.254) (layer F.Cu) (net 25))
 (segment (start 160.7817 95.25) (end 160.7817 89.8622) (width 0.254) (layer F.Cu) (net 25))
 (via (at 160.7558 87.6935) (size 0.889) (layers F.Cu B.Cu) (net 15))
 (segment (start 160.8193 87.63) (end 160.7558 87.6935) (width 0.254) (layer F.Cu) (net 15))
 (segment (start 162.052 87.63) (end 160.8193 87.63) (width 0.254) (layer F.Cu) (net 15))
 (segment (start 151.4047 87.6935) (end 151.3412 87.63) (width 0.254) (layer B.Cu) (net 15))
 (segment (start 160.7558 87.6935) (end 151.4047 87.6935) (width 0.254) (layer B.Cu) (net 15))
 (segment (start 149.86 87.63) (end 151.3412 87.63) (width 0.254) (layer B.Cu) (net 15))
 (segment (start 163.0048 92.1385) (end 162.4333 92.71) (width 0.254) (layer F.Cu) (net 2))
 (segment (start 163.0048 86.36) (end 163.0048 92.1385) (width 0.254) (layer F.Cu) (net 2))
 (segment (start 162.052 86.36) (end 163.0048 86.36) (width 0.254) (layer F.Cu) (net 2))
 (segment (start 161.6075 92.71) (end 162.4333 92.71) (width 0.254) (layer F.Cu) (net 2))
 (segment (start 165.1 86.36) (end 163.0048 86.36) (width 0.254) (layer F.Cu) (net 2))
 (segment (start 168.91 82.55) (end 165.1 86.36) (width 0.254) (layer F.Cu) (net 2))
 (segment (start 149.2513 78.6133) (end 149.86 78.6133) (width 0.254) (layer F.Cu) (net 19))
 (segment (start 148.3693 79.4953) (end 149.2513 78.6133) (width 0.254) (layer F.Cu) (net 19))
 (segment (start 148.3693 80.4799) (end 148.3693 79.4953) (width 0.254) (layer F.Cu) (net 19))
 (segment (start 149.1694 81.28) (end 148.3693 80.4799) (width 0.254) (layer F.Cu) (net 19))
 (segment (start 150.5612 81.28) (end 149.1694 81.28) (width 0.254) (layer F.Cu) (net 19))
 (segment (start 153.1012 83.82) (end 150.5612 81.28) (width 0.254) (layer F.Cu) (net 19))
 (segment (start 155.702 83.82) (end 153.1012 83.82) (width 0.254) (layer F.Cu) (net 19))
 (segment (start 149.86 77.47) (end 149.86 78.6133) (width 0.254) (layer F.Cu) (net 19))
 (segment (start 155.702 82.55) (end 156.6548 82.55) (width 0.254) (layer F.Cu) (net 21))
 (segment (start 155.2575 95.25) (end 156.0833 95.25) (width 0.254) (layer F.Cu) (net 21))
 (segment (start 156.6548 82.55) (end 157.749 82.55) (width 0.254) (layer F.Cu) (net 21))
 (segment (start 173.1016 85.9784) (end 171.45 87.63) (width 0.254) (layer F.Cu) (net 21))
 (segment (start 173.1016 79.2379) (end 173.1016 85.9784) (width 0.254) (layer F.Cu) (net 21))
 (segment (start 171.6899 77.8262) (end 173.1016 79.2379) (width 0.254) (layer F.Cu) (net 21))
 (segment (start 162.1265 77.8262) (end 171.6899 77.8262) (width 0.254) (layer F.Cu) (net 21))
 (segment (start 157.749 82.2037) (end 162.1265 77.8262) (width 0.254) (layer F.Cu) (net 21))
 (segment (start 157.749 82.55) (end 157.749 82.2037) (width 0.254) (layer F.Cu) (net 21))
 (segment (start 157.9986 82.7996) (end 157.749 82.55) (width 0.254) (layer F.Cu) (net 21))
 (segment (start 157.9986 93.6309) (end 157.9986 82.7996) (width 0.254) (layer F.Cu) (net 21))
 (segment (start 157.8396 93.7899) (end 157.9986 93.6309) (width 0.254) (layer F.Cu) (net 21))
 (segment (start 156.924 93.7899) (end 157.8396 93.7899) (width 0.254) (layer F.Cu) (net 21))
 (segment (start 156.0833 94.6306) (end 156.924 93.7899) (width 0.254) (layer F.Cu) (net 21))
 (segment (start 156.0833 95.25) (end 156.0833 94.6306) (width 0.254) (layer F.Cu) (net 21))
 (segment (start 149.2513 76.0733) (end 149.86 76.0733) (width 0.254) (layer F.Cu) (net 20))
 (segment (start 147.8574 77.4672) (end 149.2513 76.0733) (width 0.254) (layer F.Cu) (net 20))
 (segment (start 147.8574 82.5088) (end 147.8574 77.4672) (width 0.254) (layer F.Cu) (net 20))
 (segment (start 149.1351 83.7865) (end 147.8574 82.5088) (width 0.254) (layer F.Cu) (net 20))
 (segment (start 151.676 83.7865) (end 149.1351 83.7865) (width 0.254) (layer F.Cu) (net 20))
 (segment (start 154.2495 86.36) (end 151.676 83.7865) (width 0.254) (layer F.Cu) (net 20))
 (segment (start 155.702 86.36) (end 154.2495 86.36) (width 0.254) (layer F.Cu) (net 20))
 (segment (start 149.86 74.93) (end 149.86 76.0733) (width 0.254) (layer F.Cu) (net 20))
 (segment (start 154.4317 94.39) (end 154.4317 97.79) (width 0.254) (layer F.Cu) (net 22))
 (segment (start 155.0318 93.7899) (end 154.4317 94.39) (width 0.254) (layer F.Cu) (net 22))
 (segment (start 155.8883 93.7899) (end 155.0318 93.7899) (width 0.254) (layer F.Cu) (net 22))
 (segment (start 156.205 93.4732) (end 155.8883 93.7899) (width 0.254) (layer F.Cu) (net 22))
 (segment (start 156.205 89.2595) (end 156.205 93.4732) (width 0.254) (layer F.Cu) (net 22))
 (segment (start 156.6548 88.8097) (end 156.205 89.2595) (width 0.254) (layer F.Cu) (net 22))
 (segment (start 156.6548 85.09) (end 156.6548 88.8097) (width 0.254) (layer F.Cu) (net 22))
 (segment (start 155.702 85.09) (end 156.6548 85.09) (width 0.254) (layer F.Cu) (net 22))
 (segment (start 155.2575 97.79) (end 154.4317 97.79) (width 0.254) (layer F.Cu) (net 22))
 (segment (start 154.4317 101.1891) (end 154.4317 97.79) (width 0.254) (layer F.Cu) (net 22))
 (segment (start 155.1943 101.9517) (end 154.4317 101.1891) (width 0.254) (layer F.Cu) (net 22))
 (segment (start 159.8747 101.9517) (end 155.1943 101.9517) (width 0.254) (layer F.Cu) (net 22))
 (segment (start 167.4656 94.3608) (end 159.8747 101.9517) (width 0.254) (layer F.Cu) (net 22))
 (segment (start 167.4656 89.0744) (end 167.4656 94.3608) (width 0.254) (layer F.Cu) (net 22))
 (segment (start 168.91 87.63) (end 167.4656 89.0744) (width 0.254) (layer F.Cu) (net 22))
 (segment (start 149.9867 104.14) (end 149.86 104.0133) (width 0.254) (layer F.Cu) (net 10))
 (segment (start 168.91 104.14) (end 149.9867 104.14) (width 0.254) (layer F.Cu) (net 10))
 (segment (start 149.86 102.87) (end 149.86 104.0133) (width 0.254) (layer F.Cu) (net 10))
 (segment (start 138.2919 95.4769) (end 138.2919 92.71) (width 0.254) (layer B.Cu) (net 6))
 (segment (start 144.5063 101.6913) (end 138.2919 95.4769) (width 0.254) (layer B.Cu) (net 6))
 (segment (start 152.9112 101.6913) (end 144.5063 101.6913) (width 0.254) (layer B.Cu) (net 6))
 (segment (start 162.9799 111.76) (end 152.9112 101.6913) (width 0.254) (layer B.Cu) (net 6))
 (segment (start 168.91 111.76) (end 162.9799 111.76) (width 0.254) (layer B.Cu) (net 6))
 (segment (start 137.16 92.71) (end 138.2919 92.71) (width 0.254) (layer B.Cu) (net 6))
 (segment (start 139.7 92.71) (end 139.7 93.8533) (width 0.254) (layer B.Cu) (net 7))
 (segment (start 140.8433 93.8533) (end 139.7 93.8533) (width 0.254) (layer B.Cu) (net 7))
 (segment (start 146.05 99.06) (end 140.8433 93.8533) (width 0.254) (layer B.Cu) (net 7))
 (segment (start 152.8522 99.06) (end 146.05 99.06) (width 0.254) (layer B.Cu) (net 7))
 (segment (start 163.0122 109.22) (end 152.8522 99.06) (width 0.254) (layer B.Cu) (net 7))
 (segment (start 168.91 109.22) (end 163.0122 109.22) (width 0.254) (layer B.Cu) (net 7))
 (segment (start 140.8433 88.7733) (end 139.7 88.7733) (width 0.254) (layer B.Cu) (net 3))
 (segment (start 146.05 93.98) (end 140.8433 88.7733) (width 0.254) (layer B.Cu) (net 3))
 (segment (start 153.0934 93.98) (end 146.05 93.98) (width 0.254) (layer B.Cu) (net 3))
 (segment (start 161.9834 102.87) (end 153.0934 93.98) (width 0.254) (layer B.Cu) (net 3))
 (segment (start 170.18 102.87) (end 161.9834 102.87) (width 0.254) (layer B.Cu) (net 3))
 (segment (start 171.45 104.14) (end 170.18 102.87) (width 0.254) (layer B.Cu) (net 3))
 (segment (start 139.7 87.63) (end 139.7 88.7733) (width 0.254) (layer B.Cu) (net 3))
 (segment (start 139.7 90.17) (end 139.7 91.3133) (width 0.254) (layer B.Cu) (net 5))
 (segment (start 140.8433 91.3133) (end 139.7 91.3133) (width 0.254) (layer B.Cu) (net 5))
 (segment (start 146.05 96.52) (end 140.8433 91.3133) (width 0.254) (layer B.Cu) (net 5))
 (segment (start 152.3959 96.52) (end 146.05 96.52) (width 0.254) (layer B.Cu) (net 5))
 (segment (start 162.5559 106.68) (end 152.3959 96.52) (width 0.254) (layer B.Cu) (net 5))
 (segment (start 168.91 106.68) (end 162.5559 106.68) (width 0.254) (layer B.Cu) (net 5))
 (segment (start 136.4398 91.3133) (end 137.16 91.3133) (width 0.254) (layer B.Cu) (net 4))
 (segment (start 135.5112 92.2419) (end 136.4398 91.3133) (width 0.254) (layer B.Cu) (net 4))
 (segment (start 135.5112 95.7307) (end 135.5112 92.2419) (width 0.254) (layer B.Cu) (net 4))
 (segment (start 142.2538 102.4733) (end 135.5112 95.7307) (width 0.254) (layer B.Cu) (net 4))
 (segment (start 147.5035 102.4733) (end 142.2538 102.4733) (width 0.254) (layer B.Cu) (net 4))
 (segment (start 149.1702 104.14) (end 147.5035 102.4733) (width 0.254) (layer B.Cu) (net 4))
 (segment (start 152.7929 104.14) (end 149.1702 104.14) (width 0.254) (layer B.Cu) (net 4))
 (segment (start 161.5943 112.9414) (end 152.7929 104.14) (width 0.254) (layer B.Cu) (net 4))
 (segment (start 169.4111 112.9414) (end 161.5943 112.9414) (width 0.254) (layer B.Cu) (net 4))
 (segment (start 170.3067 112.0458) (end 169.4111 112.9414) (width 0.254) (layer B.Cu) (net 4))
 (segment (start 170.3067 111.76) (end 170.3067 112.0458) (width 0.254) (layer B.Cu) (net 4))
 (segment (start 171.45 111.76) (end 170.3067 111.76) (width 0.254) (layer B.Cu) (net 4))
 (segment (start 137.16 90.17) (end 137.16 91.3133) (width 0.254) (layer B.Cu) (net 4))
 (via (at 157.1625 90.5291) (size 0.889) (layers F.Cu B.Cu) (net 8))
 (segment (start 138.2919 95.4869) (end 138.2919 95.25) (width 0.254) (layer F.Cu) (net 8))
 (segment (start 139.4715 96.6665) (end 138.2919 95.4869) (width 0.254) (layer F.Cu) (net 8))
 (segment (start 140.4406 96.6665) (end 139.4715 96.6665) (width 0.254) (layer F.Cu) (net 8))
 (segment (start 147.8703 104.0962) (end 140.4406 96.6665) (width 0.254) (layer F.Cu) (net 8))
 (segment (start 147.8703 113.0087) (end 147.8703 104.0962) (width 0.254) (layer F.Cu) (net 8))
 (segment (start 149.2883 114.4267) (end 147.8703 113.0087) (width 0.254) (layer F.Cu) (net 8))
 (segment (start 149.86 114.4267) (end 149.2883 114.4267) (width 0.254) (layer F.Cu) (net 8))
 (segment (start 149.86 115.57) (end 149.86 114.4267) (width 0.254) (layer F.Cu) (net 8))
 (segment (start 137.16 95.25) (end 138.2919 95.25) (width 0.254) (layer F.Cu) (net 8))
 (segment (start 169.7109 115.57) (end 149.86 115.57) (width 0.254) (layer B.Cu) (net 8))
 (segment (start 173.6464 111.6345) (end 169.7109 115.57) (width 0.254) (layer B.Cu) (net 8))
 (segment (start 173.6464 90.0564) (end 173.6464 111.6345) (width 0.254) (layer B.Cu) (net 8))
 (segment (start 172.49 88.9) (end 173.6464 90.0564) (width 0.254) (layer B.Cu) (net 8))
 (segment (start 172.6168 88.7732) (end 172.49 88.9) (width 0.254) (layer B.Cu) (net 8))
 (segment (start 172.6168 81.1768) (end 172.6168 88.7732) (width 0.254) (layer B.Cu) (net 8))
 (segment (start 171.45 80.01) (end 172.6168 81.1768) (width 0.254) (layer B.Cu) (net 8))
 (segment (start 158.7916 88.9) (end 157.1625 90.5291) (width 0.254) (layer B.Cu) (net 8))
 (segment (start 172.49 88.9) (end 158.7916 88.9) (width 0.254) (layer B.Cu) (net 8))
 (segment (start 157.1625 92.71) (end 157.1625 90.5291) (width 0.254) (layer F.Cu) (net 8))
 (segment (start 170.2829 78.8429) (end 171.45 80.01) (width 0.254) (layer F.Cu) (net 8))
 (segment (start 164.1719 78.8429) (end 170.2829 78.8429) (width 0.254) (layer F.Cu) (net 8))
 (segment (start 163.0048 80.01) (end 164.1719 78.8429) (width 0.254) (layer F.Cu) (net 8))
 (segment (start 162.052 80.01) (end 163.0048 80.01) (width 0.254) (layer F.Cu) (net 8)))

